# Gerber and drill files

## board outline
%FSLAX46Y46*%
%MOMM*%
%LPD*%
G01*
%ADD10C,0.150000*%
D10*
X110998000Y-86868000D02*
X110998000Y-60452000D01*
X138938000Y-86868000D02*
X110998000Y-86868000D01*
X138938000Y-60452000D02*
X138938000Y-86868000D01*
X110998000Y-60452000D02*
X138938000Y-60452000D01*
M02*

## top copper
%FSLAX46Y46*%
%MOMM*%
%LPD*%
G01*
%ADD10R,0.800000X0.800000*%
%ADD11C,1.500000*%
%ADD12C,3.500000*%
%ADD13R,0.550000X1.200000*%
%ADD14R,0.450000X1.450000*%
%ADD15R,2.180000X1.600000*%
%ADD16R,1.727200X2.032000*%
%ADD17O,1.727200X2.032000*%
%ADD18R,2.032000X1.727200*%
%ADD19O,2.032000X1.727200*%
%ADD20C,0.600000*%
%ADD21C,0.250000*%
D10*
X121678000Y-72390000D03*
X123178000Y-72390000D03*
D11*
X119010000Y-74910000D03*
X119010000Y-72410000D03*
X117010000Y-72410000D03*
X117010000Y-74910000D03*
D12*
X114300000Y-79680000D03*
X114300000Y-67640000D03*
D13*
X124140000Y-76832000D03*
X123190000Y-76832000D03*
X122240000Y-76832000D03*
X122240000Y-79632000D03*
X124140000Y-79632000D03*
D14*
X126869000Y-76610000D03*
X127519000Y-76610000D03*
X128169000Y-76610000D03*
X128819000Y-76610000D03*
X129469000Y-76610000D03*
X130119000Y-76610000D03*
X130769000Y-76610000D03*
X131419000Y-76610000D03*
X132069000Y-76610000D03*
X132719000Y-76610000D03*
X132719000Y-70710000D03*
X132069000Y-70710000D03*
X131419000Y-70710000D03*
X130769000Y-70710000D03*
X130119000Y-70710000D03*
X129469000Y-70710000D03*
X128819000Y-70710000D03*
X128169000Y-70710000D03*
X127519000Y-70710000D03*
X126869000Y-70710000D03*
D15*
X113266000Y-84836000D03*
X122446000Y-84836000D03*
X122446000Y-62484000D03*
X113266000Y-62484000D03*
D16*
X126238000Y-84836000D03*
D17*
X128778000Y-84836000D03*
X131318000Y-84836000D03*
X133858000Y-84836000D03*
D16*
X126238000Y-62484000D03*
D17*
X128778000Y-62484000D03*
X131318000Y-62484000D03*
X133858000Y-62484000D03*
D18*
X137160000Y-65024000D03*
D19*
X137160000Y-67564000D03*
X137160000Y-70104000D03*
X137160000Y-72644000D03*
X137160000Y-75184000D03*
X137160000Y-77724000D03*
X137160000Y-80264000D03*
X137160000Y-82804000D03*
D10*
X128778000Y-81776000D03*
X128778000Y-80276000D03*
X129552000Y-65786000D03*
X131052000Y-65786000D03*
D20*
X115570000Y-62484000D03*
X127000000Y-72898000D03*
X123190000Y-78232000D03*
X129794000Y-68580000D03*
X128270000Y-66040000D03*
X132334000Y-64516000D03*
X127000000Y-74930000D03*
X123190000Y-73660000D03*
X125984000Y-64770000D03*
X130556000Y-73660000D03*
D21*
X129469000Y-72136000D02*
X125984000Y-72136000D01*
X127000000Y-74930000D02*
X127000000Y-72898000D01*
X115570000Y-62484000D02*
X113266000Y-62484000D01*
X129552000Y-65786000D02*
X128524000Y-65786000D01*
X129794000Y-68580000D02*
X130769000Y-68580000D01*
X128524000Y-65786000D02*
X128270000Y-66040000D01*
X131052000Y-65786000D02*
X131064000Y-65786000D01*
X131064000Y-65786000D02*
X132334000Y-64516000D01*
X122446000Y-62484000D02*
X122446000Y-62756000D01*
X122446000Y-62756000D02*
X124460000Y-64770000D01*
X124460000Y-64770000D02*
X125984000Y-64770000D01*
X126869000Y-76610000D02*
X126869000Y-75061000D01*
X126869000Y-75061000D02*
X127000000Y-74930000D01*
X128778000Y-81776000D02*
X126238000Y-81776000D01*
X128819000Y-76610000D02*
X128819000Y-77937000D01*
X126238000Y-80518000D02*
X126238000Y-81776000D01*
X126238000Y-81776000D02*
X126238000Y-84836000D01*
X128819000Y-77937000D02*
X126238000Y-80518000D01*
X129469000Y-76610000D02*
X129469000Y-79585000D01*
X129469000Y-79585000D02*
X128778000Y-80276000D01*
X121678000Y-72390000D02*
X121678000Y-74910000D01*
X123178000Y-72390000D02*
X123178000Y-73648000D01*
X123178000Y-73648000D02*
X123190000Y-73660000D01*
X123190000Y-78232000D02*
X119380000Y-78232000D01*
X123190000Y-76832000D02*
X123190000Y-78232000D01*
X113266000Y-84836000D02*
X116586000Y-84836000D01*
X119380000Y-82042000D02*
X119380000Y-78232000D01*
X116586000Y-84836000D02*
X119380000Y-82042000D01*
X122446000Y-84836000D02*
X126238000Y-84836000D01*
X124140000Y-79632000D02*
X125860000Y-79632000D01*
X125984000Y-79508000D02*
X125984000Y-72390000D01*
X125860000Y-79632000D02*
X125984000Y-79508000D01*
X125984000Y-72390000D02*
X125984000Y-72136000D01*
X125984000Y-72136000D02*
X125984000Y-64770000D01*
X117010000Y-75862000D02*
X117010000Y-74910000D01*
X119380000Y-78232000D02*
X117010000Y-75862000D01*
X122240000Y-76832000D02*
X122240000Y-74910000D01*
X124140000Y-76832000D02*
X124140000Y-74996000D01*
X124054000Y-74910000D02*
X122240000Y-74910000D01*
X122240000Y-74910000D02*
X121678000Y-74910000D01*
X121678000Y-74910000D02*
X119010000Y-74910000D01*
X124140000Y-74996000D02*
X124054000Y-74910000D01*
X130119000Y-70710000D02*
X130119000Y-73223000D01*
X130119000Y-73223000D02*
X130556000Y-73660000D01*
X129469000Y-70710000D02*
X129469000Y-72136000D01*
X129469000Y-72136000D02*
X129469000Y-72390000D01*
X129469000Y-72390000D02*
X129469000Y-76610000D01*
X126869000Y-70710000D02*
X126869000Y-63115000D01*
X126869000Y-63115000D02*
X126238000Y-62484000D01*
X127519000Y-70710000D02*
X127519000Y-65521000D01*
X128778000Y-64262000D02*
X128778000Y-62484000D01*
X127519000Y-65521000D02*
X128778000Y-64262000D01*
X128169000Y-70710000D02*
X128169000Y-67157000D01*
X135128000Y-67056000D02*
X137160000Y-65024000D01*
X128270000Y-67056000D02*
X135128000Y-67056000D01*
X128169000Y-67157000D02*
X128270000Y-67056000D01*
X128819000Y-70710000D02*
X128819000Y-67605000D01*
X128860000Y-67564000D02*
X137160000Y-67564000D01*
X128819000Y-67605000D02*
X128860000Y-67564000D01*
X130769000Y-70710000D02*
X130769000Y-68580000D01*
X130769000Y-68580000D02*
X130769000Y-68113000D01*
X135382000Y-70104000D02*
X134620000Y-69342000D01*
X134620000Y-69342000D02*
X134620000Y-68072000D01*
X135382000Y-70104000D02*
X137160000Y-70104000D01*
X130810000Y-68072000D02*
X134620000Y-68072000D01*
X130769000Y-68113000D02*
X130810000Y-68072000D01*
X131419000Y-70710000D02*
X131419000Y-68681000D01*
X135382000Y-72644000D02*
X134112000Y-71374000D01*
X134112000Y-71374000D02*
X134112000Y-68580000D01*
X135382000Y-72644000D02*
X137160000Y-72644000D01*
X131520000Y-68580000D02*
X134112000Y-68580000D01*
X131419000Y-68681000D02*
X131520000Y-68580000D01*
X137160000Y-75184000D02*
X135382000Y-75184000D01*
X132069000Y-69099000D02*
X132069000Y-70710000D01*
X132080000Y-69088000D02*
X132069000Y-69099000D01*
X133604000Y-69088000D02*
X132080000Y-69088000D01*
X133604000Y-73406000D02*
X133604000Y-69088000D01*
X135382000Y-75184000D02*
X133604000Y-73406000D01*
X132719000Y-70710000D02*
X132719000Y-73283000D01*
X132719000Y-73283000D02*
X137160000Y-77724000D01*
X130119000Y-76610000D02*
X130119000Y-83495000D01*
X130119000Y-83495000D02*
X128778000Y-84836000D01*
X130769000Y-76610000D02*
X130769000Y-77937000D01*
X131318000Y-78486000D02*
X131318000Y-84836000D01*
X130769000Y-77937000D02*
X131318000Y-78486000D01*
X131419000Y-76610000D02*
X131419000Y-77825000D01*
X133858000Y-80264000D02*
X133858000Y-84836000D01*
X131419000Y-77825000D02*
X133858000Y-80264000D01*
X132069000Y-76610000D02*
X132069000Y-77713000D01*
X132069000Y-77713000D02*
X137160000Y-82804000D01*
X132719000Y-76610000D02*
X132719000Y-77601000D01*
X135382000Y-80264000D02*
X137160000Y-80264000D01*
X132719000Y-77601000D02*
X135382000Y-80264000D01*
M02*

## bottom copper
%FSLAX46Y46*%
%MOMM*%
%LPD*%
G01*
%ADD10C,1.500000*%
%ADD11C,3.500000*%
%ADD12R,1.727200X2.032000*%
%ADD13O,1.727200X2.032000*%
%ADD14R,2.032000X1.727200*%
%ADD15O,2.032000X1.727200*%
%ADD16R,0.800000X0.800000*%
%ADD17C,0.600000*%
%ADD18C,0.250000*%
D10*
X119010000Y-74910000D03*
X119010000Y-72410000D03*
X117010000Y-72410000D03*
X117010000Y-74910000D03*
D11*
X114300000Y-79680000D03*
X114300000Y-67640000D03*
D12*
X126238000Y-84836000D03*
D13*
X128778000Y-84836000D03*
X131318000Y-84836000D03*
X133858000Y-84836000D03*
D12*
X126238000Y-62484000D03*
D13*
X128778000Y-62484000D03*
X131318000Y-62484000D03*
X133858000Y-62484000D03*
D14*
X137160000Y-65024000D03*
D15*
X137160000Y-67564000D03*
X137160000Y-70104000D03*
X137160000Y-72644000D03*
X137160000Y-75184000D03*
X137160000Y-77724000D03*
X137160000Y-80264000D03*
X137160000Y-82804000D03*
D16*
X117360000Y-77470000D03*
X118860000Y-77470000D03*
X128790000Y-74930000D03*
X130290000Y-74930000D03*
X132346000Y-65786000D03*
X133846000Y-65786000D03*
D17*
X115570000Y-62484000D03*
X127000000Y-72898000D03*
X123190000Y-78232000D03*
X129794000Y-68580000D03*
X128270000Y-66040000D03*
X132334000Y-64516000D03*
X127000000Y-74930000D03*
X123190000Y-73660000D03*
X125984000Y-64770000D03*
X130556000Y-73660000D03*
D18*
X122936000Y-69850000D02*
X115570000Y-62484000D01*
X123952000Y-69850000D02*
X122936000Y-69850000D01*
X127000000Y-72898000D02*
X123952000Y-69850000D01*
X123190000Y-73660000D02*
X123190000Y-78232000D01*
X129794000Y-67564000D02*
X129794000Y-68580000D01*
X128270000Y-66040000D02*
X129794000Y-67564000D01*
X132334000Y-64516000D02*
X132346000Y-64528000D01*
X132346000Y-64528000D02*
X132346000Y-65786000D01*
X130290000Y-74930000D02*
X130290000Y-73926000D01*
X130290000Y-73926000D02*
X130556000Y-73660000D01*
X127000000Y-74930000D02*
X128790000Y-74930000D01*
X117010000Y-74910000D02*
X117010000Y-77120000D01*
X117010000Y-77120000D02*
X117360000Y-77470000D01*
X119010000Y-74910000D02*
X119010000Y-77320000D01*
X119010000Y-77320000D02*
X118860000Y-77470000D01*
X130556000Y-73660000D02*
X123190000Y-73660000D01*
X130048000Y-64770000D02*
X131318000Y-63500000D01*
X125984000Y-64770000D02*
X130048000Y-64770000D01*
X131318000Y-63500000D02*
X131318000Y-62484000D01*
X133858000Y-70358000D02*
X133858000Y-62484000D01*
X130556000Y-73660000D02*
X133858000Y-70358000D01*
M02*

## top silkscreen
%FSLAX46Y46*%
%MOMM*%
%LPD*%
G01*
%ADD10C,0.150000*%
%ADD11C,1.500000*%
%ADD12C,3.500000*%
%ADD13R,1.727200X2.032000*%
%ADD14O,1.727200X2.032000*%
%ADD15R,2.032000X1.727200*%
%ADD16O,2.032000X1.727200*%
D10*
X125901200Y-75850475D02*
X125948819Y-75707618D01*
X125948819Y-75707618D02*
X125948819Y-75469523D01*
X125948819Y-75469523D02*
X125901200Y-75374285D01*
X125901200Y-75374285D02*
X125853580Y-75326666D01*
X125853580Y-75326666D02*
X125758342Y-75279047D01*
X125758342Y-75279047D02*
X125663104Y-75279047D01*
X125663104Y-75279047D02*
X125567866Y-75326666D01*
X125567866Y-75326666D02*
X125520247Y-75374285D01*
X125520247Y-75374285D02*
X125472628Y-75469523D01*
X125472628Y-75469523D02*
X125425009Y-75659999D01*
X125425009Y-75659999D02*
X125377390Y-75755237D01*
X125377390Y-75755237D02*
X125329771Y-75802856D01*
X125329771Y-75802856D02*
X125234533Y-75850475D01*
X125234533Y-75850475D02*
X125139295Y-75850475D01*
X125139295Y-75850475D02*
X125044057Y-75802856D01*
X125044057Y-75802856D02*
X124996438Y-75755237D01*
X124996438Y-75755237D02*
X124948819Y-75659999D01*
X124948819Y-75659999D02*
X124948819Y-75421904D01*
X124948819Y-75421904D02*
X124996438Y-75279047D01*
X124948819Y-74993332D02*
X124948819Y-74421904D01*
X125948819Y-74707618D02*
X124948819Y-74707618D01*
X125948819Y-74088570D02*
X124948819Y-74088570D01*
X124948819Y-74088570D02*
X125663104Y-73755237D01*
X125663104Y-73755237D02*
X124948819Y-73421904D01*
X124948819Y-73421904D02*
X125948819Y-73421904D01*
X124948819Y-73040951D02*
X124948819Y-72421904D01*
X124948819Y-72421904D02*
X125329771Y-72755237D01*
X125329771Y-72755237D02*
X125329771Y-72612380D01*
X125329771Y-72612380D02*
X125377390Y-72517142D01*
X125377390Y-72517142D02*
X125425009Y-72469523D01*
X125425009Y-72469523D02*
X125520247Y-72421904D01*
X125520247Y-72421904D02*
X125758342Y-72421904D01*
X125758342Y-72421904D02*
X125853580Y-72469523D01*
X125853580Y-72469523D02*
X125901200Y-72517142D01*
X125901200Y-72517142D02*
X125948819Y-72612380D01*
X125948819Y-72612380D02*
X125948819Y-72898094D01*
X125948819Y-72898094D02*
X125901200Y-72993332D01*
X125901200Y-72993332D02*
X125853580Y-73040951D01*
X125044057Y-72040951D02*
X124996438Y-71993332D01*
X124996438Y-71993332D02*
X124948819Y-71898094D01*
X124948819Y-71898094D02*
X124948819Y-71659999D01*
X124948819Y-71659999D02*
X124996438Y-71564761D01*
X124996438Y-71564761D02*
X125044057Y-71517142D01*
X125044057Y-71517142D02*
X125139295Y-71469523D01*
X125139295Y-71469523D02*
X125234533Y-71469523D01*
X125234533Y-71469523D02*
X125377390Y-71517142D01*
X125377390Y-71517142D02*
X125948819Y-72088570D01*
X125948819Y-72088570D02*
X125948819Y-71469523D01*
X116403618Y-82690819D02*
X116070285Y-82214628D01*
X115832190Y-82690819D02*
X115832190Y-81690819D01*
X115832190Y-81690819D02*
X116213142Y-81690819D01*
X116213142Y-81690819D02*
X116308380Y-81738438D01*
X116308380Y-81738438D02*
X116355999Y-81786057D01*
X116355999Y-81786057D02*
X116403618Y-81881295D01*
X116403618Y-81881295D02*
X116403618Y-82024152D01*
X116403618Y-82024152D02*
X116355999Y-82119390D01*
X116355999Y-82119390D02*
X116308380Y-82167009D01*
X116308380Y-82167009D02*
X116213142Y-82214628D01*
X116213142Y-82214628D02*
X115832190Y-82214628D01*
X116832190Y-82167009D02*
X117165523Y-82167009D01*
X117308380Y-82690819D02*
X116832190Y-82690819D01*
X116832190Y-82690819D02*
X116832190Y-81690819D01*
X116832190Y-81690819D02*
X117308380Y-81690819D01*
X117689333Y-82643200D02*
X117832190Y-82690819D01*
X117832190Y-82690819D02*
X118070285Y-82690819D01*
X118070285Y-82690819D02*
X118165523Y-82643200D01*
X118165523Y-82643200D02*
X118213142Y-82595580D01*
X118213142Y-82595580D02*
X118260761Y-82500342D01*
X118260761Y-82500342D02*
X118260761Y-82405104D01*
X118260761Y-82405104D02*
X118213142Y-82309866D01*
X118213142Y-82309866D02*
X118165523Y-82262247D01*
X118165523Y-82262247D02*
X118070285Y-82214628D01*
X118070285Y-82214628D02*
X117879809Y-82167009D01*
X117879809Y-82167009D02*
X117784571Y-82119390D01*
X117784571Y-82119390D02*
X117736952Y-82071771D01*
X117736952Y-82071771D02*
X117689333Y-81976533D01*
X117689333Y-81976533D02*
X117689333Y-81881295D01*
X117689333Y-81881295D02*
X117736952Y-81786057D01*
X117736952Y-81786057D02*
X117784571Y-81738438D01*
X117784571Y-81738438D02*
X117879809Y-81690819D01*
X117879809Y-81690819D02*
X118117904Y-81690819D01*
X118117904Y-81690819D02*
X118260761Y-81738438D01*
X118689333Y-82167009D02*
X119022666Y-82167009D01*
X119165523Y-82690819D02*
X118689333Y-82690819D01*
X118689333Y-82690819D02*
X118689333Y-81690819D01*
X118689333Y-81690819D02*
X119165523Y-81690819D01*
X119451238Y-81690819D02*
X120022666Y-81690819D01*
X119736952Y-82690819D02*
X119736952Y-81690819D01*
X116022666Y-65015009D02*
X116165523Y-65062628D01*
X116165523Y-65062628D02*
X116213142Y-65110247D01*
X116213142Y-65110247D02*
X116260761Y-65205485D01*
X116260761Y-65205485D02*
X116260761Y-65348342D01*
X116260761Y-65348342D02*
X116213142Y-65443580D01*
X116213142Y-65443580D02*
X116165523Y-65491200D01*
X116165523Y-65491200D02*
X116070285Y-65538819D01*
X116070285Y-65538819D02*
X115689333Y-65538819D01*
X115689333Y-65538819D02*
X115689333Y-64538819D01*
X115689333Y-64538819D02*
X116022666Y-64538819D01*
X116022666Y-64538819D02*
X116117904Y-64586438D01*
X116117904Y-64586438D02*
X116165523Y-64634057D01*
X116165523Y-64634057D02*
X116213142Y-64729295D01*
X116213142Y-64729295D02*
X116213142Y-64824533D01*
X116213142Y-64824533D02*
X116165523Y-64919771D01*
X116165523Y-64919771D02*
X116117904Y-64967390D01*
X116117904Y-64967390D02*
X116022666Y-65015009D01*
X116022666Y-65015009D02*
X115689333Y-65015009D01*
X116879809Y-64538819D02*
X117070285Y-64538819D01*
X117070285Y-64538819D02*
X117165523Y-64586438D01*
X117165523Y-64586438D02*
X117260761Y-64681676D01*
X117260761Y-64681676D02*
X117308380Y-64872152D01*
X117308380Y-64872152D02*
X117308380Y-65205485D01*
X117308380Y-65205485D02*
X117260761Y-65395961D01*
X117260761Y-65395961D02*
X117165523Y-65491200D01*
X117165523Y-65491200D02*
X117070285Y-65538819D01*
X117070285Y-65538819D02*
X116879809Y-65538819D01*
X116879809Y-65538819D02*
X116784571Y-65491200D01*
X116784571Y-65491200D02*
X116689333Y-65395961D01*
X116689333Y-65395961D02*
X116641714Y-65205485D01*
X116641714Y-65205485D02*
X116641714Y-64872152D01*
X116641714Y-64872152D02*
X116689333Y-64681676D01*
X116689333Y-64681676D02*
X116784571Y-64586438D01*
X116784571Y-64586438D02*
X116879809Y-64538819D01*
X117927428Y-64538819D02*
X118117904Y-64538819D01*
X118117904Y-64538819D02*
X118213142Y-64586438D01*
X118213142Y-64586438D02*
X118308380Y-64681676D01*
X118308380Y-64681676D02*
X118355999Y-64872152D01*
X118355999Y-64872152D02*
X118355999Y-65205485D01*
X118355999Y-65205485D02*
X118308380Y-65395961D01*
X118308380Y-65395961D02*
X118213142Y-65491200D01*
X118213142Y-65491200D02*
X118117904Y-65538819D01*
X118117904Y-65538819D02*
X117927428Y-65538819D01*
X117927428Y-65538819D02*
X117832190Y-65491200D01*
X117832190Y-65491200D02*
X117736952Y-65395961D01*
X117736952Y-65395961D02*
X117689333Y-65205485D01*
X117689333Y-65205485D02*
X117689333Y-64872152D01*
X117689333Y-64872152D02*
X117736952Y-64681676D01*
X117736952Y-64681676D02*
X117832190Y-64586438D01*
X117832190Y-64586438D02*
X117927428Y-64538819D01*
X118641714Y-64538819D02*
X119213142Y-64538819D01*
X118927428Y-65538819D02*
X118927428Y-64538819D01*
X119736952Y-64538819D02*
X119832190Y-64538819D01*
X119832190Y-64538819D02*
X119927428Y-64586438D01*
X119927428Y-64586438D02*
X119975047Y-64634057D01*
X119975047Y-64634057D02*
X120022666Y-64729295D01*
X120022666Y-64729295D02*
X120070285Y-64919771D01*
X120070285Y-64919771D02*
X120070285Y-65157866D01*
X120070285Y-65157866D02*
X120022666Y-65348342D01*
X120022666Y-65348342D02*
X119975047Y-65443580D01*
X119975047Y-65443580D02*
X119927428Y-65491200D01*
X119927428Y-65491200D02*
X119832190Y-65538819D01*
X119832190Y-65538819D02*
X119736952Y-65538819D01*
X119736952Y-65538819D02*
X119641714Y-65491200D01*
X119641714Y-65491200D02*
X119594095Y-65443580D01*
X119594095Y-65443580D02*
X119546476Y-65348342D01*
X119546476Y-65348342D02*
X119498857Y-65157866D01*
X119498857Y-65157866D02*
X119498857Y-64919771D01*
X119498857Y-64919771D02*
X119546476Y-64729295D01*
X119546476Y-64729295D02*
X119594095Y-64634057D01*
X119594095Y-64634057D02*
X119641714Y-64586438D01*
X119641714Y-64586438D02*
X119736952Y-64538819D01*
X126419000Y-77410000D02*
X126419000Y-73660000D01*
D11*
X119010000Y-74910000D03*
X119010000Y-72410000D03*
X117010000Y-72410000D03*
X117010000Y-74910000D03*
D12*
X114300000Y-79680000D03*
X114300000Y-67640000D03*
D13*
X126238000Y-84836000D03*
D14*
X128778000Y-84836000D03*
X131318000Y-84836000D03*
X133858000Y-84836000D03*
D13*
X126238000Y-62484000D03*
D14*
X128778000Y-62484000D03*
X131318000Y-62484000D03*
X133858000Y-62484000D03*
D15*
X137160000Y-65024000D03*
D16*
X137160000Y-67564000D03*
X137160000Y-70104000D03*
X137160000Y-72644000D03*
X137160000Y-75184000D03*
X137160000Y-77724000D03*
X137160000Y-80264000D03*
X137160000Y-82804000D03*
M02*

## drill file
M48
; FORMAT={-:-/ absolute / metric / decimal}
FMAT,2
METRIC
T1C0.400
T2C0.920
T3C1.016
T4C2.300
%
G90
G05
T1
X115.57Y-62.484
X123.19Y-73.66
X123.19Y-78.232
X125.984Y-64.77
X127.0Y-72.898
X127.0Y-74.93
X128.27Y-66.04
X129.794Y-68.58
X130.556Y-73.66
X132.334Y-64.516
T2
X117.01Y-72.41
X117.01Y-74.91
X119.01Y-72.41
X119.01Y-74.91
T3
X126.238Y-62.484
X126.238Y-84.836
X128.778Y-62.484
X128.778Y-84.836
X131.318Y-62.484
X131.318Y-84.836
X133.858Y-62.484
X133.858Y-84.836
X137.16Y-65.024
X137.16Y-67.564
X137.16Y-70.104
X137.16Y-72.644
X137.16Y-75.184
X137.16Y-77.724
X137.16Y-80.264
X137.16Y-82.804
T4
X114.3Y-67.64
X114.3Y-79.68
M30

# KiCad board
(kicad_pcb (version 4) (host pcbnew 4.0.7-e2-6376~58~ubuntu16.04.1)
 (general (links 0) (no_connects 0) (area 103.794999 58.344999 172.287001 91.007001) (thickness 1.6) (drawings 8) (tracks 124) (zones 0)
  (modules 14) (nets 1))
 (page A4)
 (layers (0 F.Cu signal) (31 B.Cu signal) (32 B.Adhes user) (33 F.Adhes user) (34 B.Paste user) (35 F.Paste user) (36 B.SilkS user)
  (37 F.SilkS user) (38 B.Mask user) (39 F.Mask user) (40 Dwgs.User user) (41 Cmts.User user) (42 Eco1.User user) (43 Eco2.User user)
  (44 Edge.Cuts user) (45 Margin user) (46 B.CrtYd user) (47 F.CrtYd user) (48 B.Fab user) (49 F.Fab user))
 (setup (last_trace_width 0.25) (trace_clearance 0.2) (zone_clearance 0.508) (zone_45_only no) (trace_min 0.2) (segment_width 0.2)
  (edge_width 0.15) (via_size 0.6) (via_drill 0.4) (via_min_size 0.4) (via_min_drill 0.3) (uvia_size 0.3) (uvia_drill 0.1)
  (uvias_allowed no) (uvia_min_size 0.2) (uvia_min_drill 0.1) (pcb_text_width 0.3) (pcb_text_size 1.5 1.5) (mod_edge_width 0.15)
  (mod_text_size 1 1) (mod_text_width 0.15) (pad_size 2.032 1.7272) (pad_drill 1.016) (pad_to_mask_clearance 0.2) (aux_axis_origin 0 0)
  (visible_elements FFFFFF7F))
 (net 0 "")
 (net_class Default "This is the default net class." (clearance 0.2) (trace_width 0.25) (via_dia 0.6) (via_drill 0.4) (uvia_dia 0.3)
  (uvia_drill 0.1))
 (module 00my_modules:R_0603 (layer F.Cu) (at 122.428 72.39)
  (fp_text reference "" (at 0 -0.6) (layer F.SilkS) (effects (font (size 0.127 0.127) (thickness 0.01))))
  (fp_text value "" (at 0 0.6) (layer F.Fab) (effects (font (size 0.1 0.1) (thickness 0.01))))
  (pad 1 smd rect (at -0.75 0) (size 0.8 0.8) (layers F.Cu F.Paste F.Mask))
  (pad 2 smd rect (at 0.75 0) (size 0.8 0.8) (layers F.Cu F.Paste F.Mask)))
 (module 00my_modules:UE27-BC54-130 (layer F.Cu) (at 114.3 73.66 270)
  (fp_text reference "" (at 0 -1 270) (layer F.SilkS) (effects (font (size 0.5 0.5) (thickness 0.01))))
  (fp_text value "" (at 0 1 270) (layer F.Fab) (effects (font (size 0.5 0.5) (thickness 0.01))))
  (pad 5V thru_hole circle (at 1.25 -4.71 270) (size 1.5 1.5) (drill 0.92) (layers *.Cu *.Mask F.SilkS))
  (pad - thru_hole circle (at -1.25 -4.71 270) (size 1.5 1.5) (drill 0.92) (layers *.Cu *.Mask F.SilkS))
  (pad + thru_hole circle (at -1.25 -2.71 270) (size 1.5 1.5) (drill 0.92) (layers *.Cu *.Mask F.SilkS))
  (pad GND thru_hole circle (at 1.25 -2.71 270) (size 1.5 1.5) (drill 0.92) (layers *.Cu *.Mask F.SilkS))
  (pad X thru_hole circle (at 6.02 0 270) (size 3.5 3.5) (drill 2.3) (layers *.Cu *.Mask F.SilkS))
  (pad X thru_hole circle (at -6.02 0 270) (size 3.5 3.5) (drill 2.3) (layers *.Cu *.Mask F.SilkS)))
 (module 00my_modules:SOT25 (layer F.Cu) (at 123.19 78.232 270)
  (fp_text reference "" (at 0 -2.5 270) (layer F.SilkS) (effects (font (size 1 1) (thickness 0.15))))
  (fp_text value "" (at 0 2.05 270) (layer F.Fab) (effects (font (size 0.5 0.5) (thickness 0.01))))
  (pad VIN smd rect (at -1.4 -0.95 270) (size 1.2 0.55) (layers F.Cu F.Paste F.Mask))
  (pad GND smd rect (at -1.4 0 270) (size 1.2 0.55) (layers F.Cu F.Paste F.Mask))
  (pad EN smd rect (at -1.4 0.95 270) (size 1.2 0.55) (layers F.Cu F.Paste F.Mask))
  (pad NC smd rect (at 1.4 0.95 270) (size 1.2 0.55) (layers F.Cu F.Paste F.Mask))
  (pad VOUT smd rect (at 1.4 -0.95 270) (size 1.2 0.55) (layers F.Cu F.Paste F.Mask)))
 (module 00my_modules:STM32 (layer F.Cu) (at 129.794 73.66 90)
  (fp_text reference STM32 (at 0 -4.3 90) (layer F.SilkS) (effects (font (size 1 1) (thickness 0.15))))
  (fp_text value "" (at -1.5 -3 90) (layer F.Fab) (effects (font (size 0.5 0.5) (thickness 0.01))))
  (fp_line (start -3.75 -3.375) (end 0 -3.375) (layer F.SilkS) (width 0.15))
  (pad BOOT smd rect (at -2.95 -2.925 90) (size 1.45 0.45) (layers F.Cu F.Paste F.Mask))
  (pad 2 smd rect (at -2.95 -2.275 90) (size 1.45 0.45) (layers F.Cu F.Paste F.Mask))
  (pad 3 smd rect (at -2.95 -1.625 90) (size 1.45 0.45) (layers F.Cu F.Paste F.Mask))
  (pad NRST smd rect (at -2.95 -0.975 90) (size 1.45 0.45) (layers F.Cu F.Paste F.Mask))
  (pad VCC smd rect (at -2.95 -0.325 90) (size 1.45 0.45) (layers F.Cu F.Paste F.Mask))
  (pad PA0 smd rect (at -2.95 0.325 90) (size 1.45 0.45) (layers F.Cu F.Paste F.Mask))
  (pad PA1 smd rect (at -2.95 0.975 90) (size 1.45 0.45) (layers F.Cu F.Paste F.Mask))
  (pad PA2 smd rect (at -2.95 1.625 90) (size 1.45 0.45) (layers F.Cu F.Paste F.Mask))
  (pad PA3 smd rect (at -2.95 2.275 90) (size 1.45 0.45) (layers F.Cu F.Paste F.Mask))
  (pad PA4 smd rect (at -2.95 2.925 90) (size 1.45 0.45) (layers F.Cu F.Paste F.Mask))
  (pad PA5 smd rect (at 2.95 2.925 90) (size 1.45 0.45) (layers F.Cu F.Paste F.Mask))
  (pad PA6 smd rect (at 2.95 2.275 90) (size 1.45 0.45) (layers F.Cu F.Paste F.Mask))
  (pad PA7 smd rect (at 2.95 1.625 90) (size 1.45 0.45) (layers F.Cu F.Paste F.Mask))
  (pad PB1 smd rect (at 2.95 0.975 90) (size 1.45 0.45) (layers F.Cu F.Paste F.Mask))
  (pad GND smd rect (at 2.95 0.325 90) (size 1.45 0.45) (layers F.Cu F.Paste F.Mask))
  (pad VCC smd rect (at 2.95 -0.325 90) (size 1.45 0.45) (layers F.Cu F.Paste F.Mask))
  (pad TX smd rect (at 2.95 -0.975 90) (size 1.45 0.45) (layers F.Cu F.Paste F.Mask))
  (pad RX smd rect (at 2.95 -1.625 90) (size 1.45 0.45) (layers F.Cu F.Paste F.Mask))
  (pad DIO smd rect (at 2.95 -2.275 90) (size 1.45 0.45) (layers F.Cu F.Paste F.Mask))
  (pad CLK smd rect (at 2.95 -2.925 90) (size 1.45 0.45) (layers F.Cu F.Paste F.Mask)))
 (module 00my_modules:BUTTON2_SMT (layer F.Cu) (at 117.856 84.836)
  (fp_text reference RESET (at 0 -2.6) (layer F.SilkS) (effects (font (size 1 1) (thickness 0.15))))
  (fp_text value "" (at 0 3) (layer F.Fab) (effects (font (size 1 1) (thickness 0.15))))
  (pad GND smd rect (at -4.59 0) (size 2.18 1.6) (layers F.Cu F.Paste F.Mask))
  (pad NRST smd rect (at 4.59 0) (size 2.18 1.6) (layers F.Cu F.Paste F.Mask)))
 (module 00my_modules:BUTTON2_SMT (layer F.Cu) (at 117.856 62.484 180)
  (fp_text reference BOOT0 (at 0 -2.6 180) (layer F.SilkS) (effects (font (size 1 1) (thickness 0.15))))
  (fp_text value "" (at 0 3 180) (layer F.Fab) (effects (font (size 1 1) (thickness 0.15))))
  (pad VCC smd rect (at -4.59 0 180) (size 2.18 1.6) (layers F.Cu F.Paste F.Mask))
  (pad BOOT smd rect (at 4.59 0 180) (size 2.18 1.6) (layers F.Cu F.Paste F.Mask)))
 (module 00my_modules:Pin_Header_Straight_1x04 (layer F.Cu) (at 126.238 84.836 90)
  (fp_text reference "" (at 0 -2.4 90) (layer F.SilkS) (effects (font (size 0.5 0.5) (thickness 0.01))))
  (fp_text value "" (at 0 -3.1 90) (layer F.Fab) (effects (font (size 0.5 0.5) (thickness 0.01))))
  (pad RST thru_hole rect (at 0 0 90) (size 2.032 1.7272) (drill 1.016) (layers *.Cu *.Mask F.SilkS))
  (pad PA0 thru_hole oval (at 0 2.54 90) (size 2.032 1.7272) (drill 1.016) (layers *.Cu *.Mask F.SilkS))
  (pad PA1 thru_hole oval (at 0 5.08 90) (size 2.032 1.7272) (drill 1.016) (layers *.Cu *.Mask F.SilkS))
  (pad PA2 thru_hole oval (at 0 7.62 90) (size 2.032 1.7272) (drill 1.016) (layers *.Cu *.Mask F.SilkS)))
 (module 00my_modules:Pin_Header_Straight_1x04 (layer F.Cu) (at 126.238 62.484 90)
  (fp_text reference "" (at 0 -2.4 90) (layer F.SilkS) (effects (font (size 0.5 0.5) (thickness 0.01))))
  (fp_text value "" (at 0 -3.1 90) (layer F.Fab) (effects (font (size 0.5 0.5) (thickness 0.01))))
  (pad CLK thru_hole rect (at 0 0 90) (size 2.032 1.7272) (drill 1.016) (layers *.Cu *.Mask F.SilkS))
  (pad DIO thru_hole oval (at 0 2.54 90) (size 2.032 1.7272) (drill 1.016) (layers *.Cu *.Mask F.SilkS))
  (pad VCC thru_hole oval (at 0 5.08 90) (size 2.032 1.7272) (drill 1.016) (layers *.Cu *.Mask F.SilkS))
  (pad GND thru_hole oval (at 0 7.62 90) (size 2.032 1.7272) (drill 1.016) (layers *.Cu *.Mask F.SilkS)))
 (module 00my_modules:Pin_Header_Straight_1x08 (layer F.Cu) (at 137.16 65.024)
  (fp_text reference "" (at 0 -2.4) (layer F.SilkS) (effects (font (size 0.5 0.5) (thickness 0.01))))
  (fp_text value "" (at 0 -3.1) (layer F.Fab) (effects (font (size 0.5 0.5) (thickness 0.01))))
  (pad RX thru_hole rect (at 0 0) (size 2.032 1.7272) (drill 1.016) (layers *.Cu *.Mask F.SilkS))
  (pad TX thru_hole oval (at 0 2.54) (size 2.032 1.7272) (drill 1.016) (layers *.Cu *.Mask F.SilkS))
  (pad PB1 thru_hole oval (at 0 5.08) (size 2.032 1.7272) (drill 1.016) (layers *.Cu *.Mask F.SilkS))
  (pad PA7 thru_hole oval (at 0 7.62) (size 2.032 1.7272) (drill 1.016) (layers *.Cu *.Mask F.SilkS))
  (pad PA6 thru_hole oval (at 0 10.16) (size 2.032 1.7272) (drill 1.016) (layers *.Cu *.Mask F.SilkS))
  (pad PA5 thru_hole oval (at 0 12.7) (size 2.032 1.7272) (drill 1.016) (layers *.Cu *.Mask F.SilkS))
  (pad PA4 thru_hole oval (at 0 15.24) (size 2.032 1.7272) (drill 1.016) (layers *.Cu *.Mask F.SilkS))
  (pad PA3 thru_hole oval (at 0 17.78) (size 2.032 1.7272) (drill 1.016) (layers *.Cu *.Mask F.SilkS)))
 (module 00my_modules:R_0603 (layer B.Cu) (at 118.11 77.47)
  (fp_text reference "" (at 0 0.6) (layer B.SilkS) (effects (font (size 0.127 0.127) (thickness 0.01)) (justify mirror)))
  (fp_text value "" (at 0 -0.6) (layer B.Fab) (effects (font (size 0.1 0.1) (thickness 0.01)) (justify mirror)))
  (pad 1 smd rect (at -0.75 0) (size 0.8 0.8) (layers B.Cu B.Paste B.Mask))
  (pad 2 smd rect (at 0.75 0) (size 0.8 0.8) (layers B.Cu B.Paste B.Mask)))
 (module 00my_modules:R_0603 (layer F.Cu) (at 128.778 81.026 90)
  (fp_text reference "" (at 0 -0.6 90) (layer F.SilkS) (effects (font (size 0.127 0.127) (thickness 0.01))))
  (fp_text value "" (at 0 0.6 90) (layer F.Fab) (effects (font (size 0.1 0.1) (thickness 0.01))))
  (pad 1 smd rect (at -0.75 0 90) (size 0.8 0.8) (layers F.Cu F.Paste F.Mask))
  (pad 2 smd rect (at 0.75 0 90) (size 0.8 0.8) (layers F.Cu F.Paste F.Mask)))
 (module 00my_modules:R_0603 (layer B.Cu) (at 129.54 74.93)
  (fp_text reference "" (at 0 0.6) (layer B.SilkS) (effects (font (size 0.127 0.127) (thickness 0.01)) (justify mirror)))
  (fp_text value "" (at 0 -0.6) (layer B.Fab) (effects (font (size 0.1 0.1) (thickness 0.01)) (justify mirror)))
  (pad 1 smd rect (at -0.75 0) (size 0.8 0.8) (layers B.Cu B.Paste B.Mask))
  (pad 2 smd rect (at 0.75 0) (size 0.8 0.8) (layers B.Cu B.Paste B.Mask)))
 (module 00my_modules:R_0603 (layer F.Cu) (at 130.302 65.786)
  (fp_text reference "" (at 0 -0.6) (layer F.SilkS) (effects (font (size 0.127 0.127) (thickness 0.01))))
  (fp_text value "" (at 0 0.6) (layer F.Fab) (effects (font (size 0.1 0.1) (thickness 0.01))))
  (pad 1 smd rect (at -0.75 0) (size 0.8 0.8) (layers F.Cu F.Paste F.Mask))
  (pad 2 smd rect (at 0.75 0) (size 0.8 0.8) (layers F.Cu F.Paste F.Mask)))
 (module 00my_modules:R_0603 (layer B.Cu) (at 133.096 65.786)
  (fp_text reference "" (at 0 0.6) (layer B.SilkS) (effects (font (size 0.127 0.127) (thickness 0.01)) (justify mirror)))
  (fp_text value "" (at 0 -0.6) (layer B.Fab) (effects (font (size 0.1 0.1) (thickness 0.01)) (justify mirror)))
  (pad 1 smd rect (at -0.75 0) (size 0.8 0.8) (layers B.Cu B.Paste B.Mask))
  (pad 2 smd rect (at 0.75 0) (size 0.8 0.8) (layers B.Cu B.Paste B.Mask)))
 (gr_line (start 110.998 86.868) (end 110.998 60.452) (angle 90) (layer Edge.Cuts) (width 0.15))
 (gr_line (start 138.938 86.868) (end 110.998 86.868) (angle 90) (layer Edge.Cuts) (width 0.15))
 (gr_line (start 138.938 60.452) (end 138.938 86.868) (angle 90) (layer Edge.Cuts) (width 0.15))
 (gr_line (start 110.998 60.452) (end 138.938 60.452) (angle 90) (layer Edge.Cuts) (width 0.15))
 (segment (start 129.469 72.136) (end 125.984 72.136) (width 0.25) (layer F.Cu) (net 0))
 (segment (start 127 74.93) (end 127 72.898) (width 0.25) (layer F.Cu) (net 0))
 (segment (start 115.57 62.484) (end 113.266 62.484) (width 0.25) (layer F.Cu) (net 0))
 (via (at 115.57 62.484) (size 0.6) (drill 0.4) (layers F.Cu B.Cu) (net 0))
 (segment (start 122.936 69.85) (end 115.57 62.484) (width 0.25) (layer B.Cu) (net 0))
 (segment (start 123.952 69.85) (end 122.936 69.85) (width 0.25) (layer B.Cu) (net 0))
 (segment (start 127 72.898) (end 123.952 69.85) (width 0.25) (layer B.Cu) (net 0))
 (via (at 127 72.898) (size 0.6) (drill 0.4) (layers F.Cu B.Cu) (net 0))
 (segment (start 123.19 73.66) (end 123.19 78.232) (width 0.25) (layer B.Cu) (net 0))
 (via (at 123.19 78.232) (size 0.6) (drill 0.4) (layers F.Cu B.Cu) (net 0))
 (segment (start 129.552 65.786) (end 128.524 65.786) (width 0.25) (layer F.Cu) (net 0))
 (segment (start 129.794 68.58) (end 130.769 68.58) (width 0.25) (layer F.Cu) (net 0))
 (via (at 129.794 68.58) (size 0.6) (drill 0.4) (layers F.Cu B.Cu) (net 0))
 (segment (start 129.794 67.564) (end 129.794 68.58) (width 0.25) (layer B.Cu) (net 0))
 (segment (start 128.27 66.04) (end 129.794 67.564) (width 0.25) (layer B.Cu) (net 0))
 (via (at 128.27 66.04) (size 0.6) (drill 0.4) (layers F.Cu B.Cu) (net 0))
 (segment (start 128.524 65.786) (end 128.27 66.04) (width 0.25) (layer F.Cu) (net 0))
 (segment (start 131.052 65.786) (end 131.064 65.786) (width 0.25) (layer F.Cu) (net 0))
 (segment (start 131.064 65.786) (end 132.334 64.516) (width 0.25) (layer F.Cu) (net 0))
 (via (at 132.334 64.516) (size 0.6) (drill 0.4) (layers F.Cu B.Cu) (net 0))
 (segment (start 132.334 64.516) (end 132.346 64.528) (width 0.25) (layer B.Cu) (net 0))
 (segment (start 132.346 64.528) (end 132.346 65.786) (width 0.25) (layer B.Cu) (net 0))
 (segment (start 122.446 62.484) (end 122.446 62.756) (width 0.25) (layer F.Cu) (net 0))
 (segment (start 122.446 62.756) (end 124.46 64.77) (width 0.25) (layer F.Cu) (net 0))
 (segment (start 124.46 64.77) (end 125.984 64.77) (width 0.25) (layer F.Cu) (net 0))
 (segment (start 130.29 74.93) (end 130.29 73.926) (width 0.25) (layer B.Cu) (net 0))
 (segment (start 130.29 73.926) (end 130.556 73.66) (width 0.25) (layer B.Cu) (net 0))
 (segment (start 126.869 76.61) (end 126.869 75.061) (width 0.25) (layer F.Cu) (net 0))
 (segment (start 127 74.93) (end 128.79 74.93) (width 0.25) (layer B.Cu) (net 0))
 (via (at 127 74.93) (size 0.6) (drill 0.4) (layers F.Cu B.Cu) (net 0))
 (segment (start 126.869 75.061) (end 127 74.93) (width 0.25) (layer F.Cu) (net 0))
 (segment (start 128.778 81.776) (end 126.238 81.776) (width 0.25) (layer F.Cu) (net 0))
 (segment (start 128.819 76.61) (end 128.819 77.937) (width 0.25) (layer F.Cu) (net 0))
 (segment (start 126.238 80.518) (end 126.238 81.776) (width 0.25) (layer F.Cu) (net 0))
 (segment (start 126.238 81.776) (end 126.238 84.836) (width 0.25) (layer F.Cu) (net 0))
 (segment (start 128.819 77.937) (end 126.238 80.518) (width 0.25) (layer F.Cu) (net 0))
 (segment (start 129.469 76.61) (end 129.469 79.585) (width 0.25) (layer F.Cu) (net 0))
 (segment (start 129.469 79.585) (end 128.778 80.276) (width 0.25) (layer F.Cu) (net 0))
 (segment (start 117.01 74.91) (end 117.01 77.12) (width 0.25) (layer B.Cu) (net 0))
 (segment (start 117.01 77.12) (end 117.36 77.47) (width 0.25) (layer B.Cu) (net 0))
 (segment (start 119.01 74.91) (end 119.01 77.32) (width 0.25) (layer B.Cu) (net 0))
 (segment (start 119.01 77.32) (end 118.86 77.47) (width 0.25) (layer B.Cu) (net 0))
 (segment (start 121.678 72.39) (end 121.678 74.91) (width 0.25) (layer F.Cu) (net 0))
 (segment (start 123.178 72.39) (end 123.178 73.648) (width 0.25) (layer F.Cu) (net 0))
 (segment (start 123.178 73.648) (end 123.19 73.66) (width 0.25) (layer F.Cu) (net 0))
 (segment (start 130.556 73.66) (end 123.19 73.66) (width 0.25) (layer B.Cu) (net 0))
 (segment (start 123.19 78.232) (end 119.38 78.232) (width 0.25) (layer F.Cu) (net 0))
 (segment (start 123.19 76.832) (end 123.19 78.232) (width 0.25) (layer F.Cu) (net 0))
 (via (at 123.19 73.66) (size 0.6) (drill 0.4) (layers F.Cu B.Cu) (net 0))
 (segment (start 113.266 84.836) (end 116.586 84.836) (width 0.25) (layer F.Cu) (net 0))
 (segment (start 119.38 82.042) (end 119.38 78.232) (width 0.25) (layer F.Cu) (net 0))
 (segment (start 116.586 84.836) (end 119.38 82.042) (width 0.25) (layer F.Cu) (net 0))
 (segment (start 122.446 84.836) (end 126.238 84.836) (width 0.25) (layer F.Cu) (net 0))
 (segment (start 124.14 79.632) (end 125.86 79.632) (width 0.25) (layer F.Cu) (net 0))
 (segment (start 125.984 79.508) (end 125.984 72.39) (width 0.25) (layer F.Cu) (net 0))
 (segment (start 125.86 79.632) (end 125.984 79.508) (width 0.25) (layer F.Cu) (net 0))
 (segment (start 125.984 72.39) (end 125.984 72.136) (width 0.25) (layer F.Cu) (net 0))
 (segment (start 125.984 72.136) (end 125.984 64.77) (width 0.25) (layer F.Cu) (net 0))
 (segment (start 117.01 75.862) (end 117.01 74.91) (width 0.25) (layer F.Cu) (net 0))
 (segment (start 119.38 78.232) (end 117.01 75.862) (width 0.25) (layer F.Cu) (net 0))
 (segment (start 122.24 76.832) (end 122.24 74.91) (width 0.25) (layer F.Cu) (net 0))
 (segment (start 124.14 76.832) (end 124.14 74.996) (width 0.25) (layer F.Cu) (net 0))
 (segment (start 124.054 74.91) (end 122.24 74.91) (width 0.25) (layer F.Cu) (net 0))
 (segment (start 122.24 74.91) (end 121.678 74.91) (width 0.25) (layer F.Cu) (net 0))
 (segment (start 121.678 74.91) (end 119.01 74.91) (width 0.25) (layer F.Cu) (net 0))
 (segment (start 124.14 74.996) (end 124.054 74.91) (width 0.25) (layer F.Cu) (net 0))
 (segment (start 130.048 64.77) (end 131.318 63.5) (width 0.25) (layer B.Cu) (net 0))
 (segment (start 125.984 64.77) (end 130.048 64.77) (width 0.25) (layer B.Cu) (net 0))
 (via (at 125.984 64.77) (size 0.6) (drill 0.4) (layers F.Cu B.Cu) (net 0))
 (segment (start 131.318 63.5) (end 131.318 62.484) (width 0.25) (layer B.Cu) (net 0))
 (segment (start 130.119 70.71) (end 130.119 73.223) (width 0.25) (layer F.Cu) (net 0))
 (segment (start 133.858 70.358) (end 133.858 62.484) (width 0.25) (layer B.Cu) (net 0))
 (segment (start 130.556 73.66) (end 133.858 70.358) (width 0.25) (layer B.Cu) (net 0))
 (via (at 130.556 73.66) (size 0.6) (drill 0.4) (layers F.Cu B.Cu) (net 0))
 (segment (start 130.119 73.223) (end 130.556 73.66) (width 0.25) (layer F.Cu) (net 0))
 (segment (start 129.469 70.71) (end 129.469 72.136) (width 0.25) (layer F.Cu) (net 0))
 (segment (start 129.469 72.136) (end 129.469 72.39) (width 0.25) (layer F.Cu) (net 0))
 (segment (start 129.469 72.39) (end 129.469 76.61) (width 0.25) (layer F.Cu) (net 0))
 (segment (start 126.869 70.71) (end 126.869 63.115) (width 0.25) (layer F.Cu) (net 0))
 (segment (start 126.869 63.115) (end 126.238 62.484) (width 0.25) (layer F.Cu) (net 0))
 (segment (start 127.519 70.71) (end 127.519 65.521) (width 0.25) (layer F.Cu) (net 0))
 (segment (start 128.778 64.262) (end 128.778 62.484) (width 0.25) (layer F.Cu) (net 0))
 (segment (start 127.519 65.521) (end 128.778 64.262) (width 0.25) (layer F.Cu) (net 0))
 (segment (start 128.169 70.71) (end 128.169 67.157) (width 0.25) (layer F.Cu) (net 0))
 (segment (start 135.128 67.056) (end 137.16 65.024) (width 0.25) (layer F.Cu) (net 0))
 (segment (start 128.27 67.056) (end 135.128 67.056) (width 0.25) (layer F.Cu) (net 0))
 (segment (start 128.169 67.157) (end 128.27 67.056) (width 0.25) (layer F.Cu) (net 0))
 (segment (start 128.819 70.71) (end 128.819 67.605) (width 0.25) (layer F.Cu) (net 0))
 (segment (start 128.86 67.564) (end 137.16 67.564) (width 0.25) (layer F.Cu) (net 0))
 (segment (start 128.819 67.605) (end 128.86 67.564) (width 0.25) (layer F.Cu) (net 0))
 (segment (start 130.769 70.71) (end 130.769 68.58) (width 0.25) (layer F.Cu) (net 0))
 (segment (start 130.769 68.58) (end 130.769 68.113) (width 0.25) (layer F.Cu) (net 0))
 (segment (start 135.382 70.104) (end 134.62 69.342) (width 0.25) (layer F.Cu) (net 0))
 (segment (start 134.62 69.342) (end 134.62 68.072) (width 0.25) (layer F.Cu) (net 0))
 (segment (start 135.382 70.104) (end 137.16 70.104) (width 0.25) (layer F.Cu) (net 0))
 (segment (start 130.81 68.072) (end 134.62 68.072) (width 0.25) (layer F.Cu) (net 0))
 (segment (start 130.769 68.113) (end 130.81 68.072) (width 0.25) (layer F.Cu) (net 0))
 (segment (start 131.419 70.71) (end 131.419 68.681) (width 0.25) (layer F.Cu) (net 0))
 (segment (start 135.382 72.644) (end 134.112 71.374) (width 0.25) (layer F.Cu) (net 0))
 (segment (start 134.112 71.374) (end 134.112 68.58) (width 0.25) (layer F.Cu) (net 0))
 (segment (start 135.382 72.644) (end 137.16 72.644) (width 0.25) (layer F.Cu) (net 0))
 (segment (start 131.52 68.58) (end 134.112 68.58) (width 0.25) (layer F.Cu) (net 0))
 (segment (start 131.419 68.681) (end 131.52 68.58) (width 0.25) (layer F.Cu) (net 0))
 (segment (start 137.16 75.184) (end 135.382 75.184) (width 0.25) (layer F.Cu) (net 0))
 (segment (start 132.069 69.099) (end 132.069 70.71) (width 0.25) (layer F.Cu) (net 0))
 (segment (start 132.08 69.088) (end 132.069 69.099) (width 0.25) (layer F.Cu) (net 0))
 (segment (start 133.604 69.088) (end 132.08 69.088) (width 0.25) (layer F.Cu) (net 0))
 (segment (start 133.604 73.406) (end 133.604 69.088) (width 0.25) (layer F.Cu) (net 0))
 (segment (start 135.382 75.184) (end 133.604 73.406) (width 0.25) (layer F.Cu) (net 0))
 (segment (start 132.719 70.71) (end 132.719 73.283) (width 0.25) (layer F.Cu) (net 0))
 (segment (start 132.719 73.283) (end 137.16 77.724) (width 0.25) (layer F.Cu) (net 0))
 (segment (start 130.119 76.61) (end 130.119 83.495) (width 0.25) (layer F.Cu) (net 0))
 (segment (start 130.119 83.495) (end 128.778 84.836) (width 0.25) (layer F.Cu) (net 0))
 (segment (start 130.769 76.61) (end 130.769 77.937) (width 0.25) (layer F.Cu) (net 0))
 (segment (start 131.318 78.486) (end 131.318 84.836) (width 0.25) (layer F.Cu) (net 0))
 (segment (start 130.769 77.937) (end 131.318 78.486) (width 0.25) (layer F.Cu) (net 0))
 (segment (start 131.419 76.61) (end 131.419 77.825) (width 0.25) (layer F.Cu) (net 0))
 (segment (start 133.858 80.264) (end 133.858 84.836) (width 0.25) (layer F.Cu) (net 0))
 (segment (start 131.419 77.825) (end 133.858 80.264) (width 0.25) (layer F.Cu) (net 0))
 (segment (start 132.069 76.61) (end 132.069 77.713) (width 0.25) (layer F.Cu) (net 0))
 (segment (start 132.069 77.713) (end 137.16 82.804) (width 0.25) (layer F.Cu) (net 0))
 (segment (start 132.719 76.61) (end 132.719 77.601) (width 0.25) (layer F.Cu) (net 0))
 (segment (start 135.382 80.264) (end 137.16 80.264) (width 0.25) (layer F.Cu) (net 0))
 (segment (start 132.719 77.601) (end 135.382 80.264) (width 0.25) (layer F.Cu) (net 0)))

